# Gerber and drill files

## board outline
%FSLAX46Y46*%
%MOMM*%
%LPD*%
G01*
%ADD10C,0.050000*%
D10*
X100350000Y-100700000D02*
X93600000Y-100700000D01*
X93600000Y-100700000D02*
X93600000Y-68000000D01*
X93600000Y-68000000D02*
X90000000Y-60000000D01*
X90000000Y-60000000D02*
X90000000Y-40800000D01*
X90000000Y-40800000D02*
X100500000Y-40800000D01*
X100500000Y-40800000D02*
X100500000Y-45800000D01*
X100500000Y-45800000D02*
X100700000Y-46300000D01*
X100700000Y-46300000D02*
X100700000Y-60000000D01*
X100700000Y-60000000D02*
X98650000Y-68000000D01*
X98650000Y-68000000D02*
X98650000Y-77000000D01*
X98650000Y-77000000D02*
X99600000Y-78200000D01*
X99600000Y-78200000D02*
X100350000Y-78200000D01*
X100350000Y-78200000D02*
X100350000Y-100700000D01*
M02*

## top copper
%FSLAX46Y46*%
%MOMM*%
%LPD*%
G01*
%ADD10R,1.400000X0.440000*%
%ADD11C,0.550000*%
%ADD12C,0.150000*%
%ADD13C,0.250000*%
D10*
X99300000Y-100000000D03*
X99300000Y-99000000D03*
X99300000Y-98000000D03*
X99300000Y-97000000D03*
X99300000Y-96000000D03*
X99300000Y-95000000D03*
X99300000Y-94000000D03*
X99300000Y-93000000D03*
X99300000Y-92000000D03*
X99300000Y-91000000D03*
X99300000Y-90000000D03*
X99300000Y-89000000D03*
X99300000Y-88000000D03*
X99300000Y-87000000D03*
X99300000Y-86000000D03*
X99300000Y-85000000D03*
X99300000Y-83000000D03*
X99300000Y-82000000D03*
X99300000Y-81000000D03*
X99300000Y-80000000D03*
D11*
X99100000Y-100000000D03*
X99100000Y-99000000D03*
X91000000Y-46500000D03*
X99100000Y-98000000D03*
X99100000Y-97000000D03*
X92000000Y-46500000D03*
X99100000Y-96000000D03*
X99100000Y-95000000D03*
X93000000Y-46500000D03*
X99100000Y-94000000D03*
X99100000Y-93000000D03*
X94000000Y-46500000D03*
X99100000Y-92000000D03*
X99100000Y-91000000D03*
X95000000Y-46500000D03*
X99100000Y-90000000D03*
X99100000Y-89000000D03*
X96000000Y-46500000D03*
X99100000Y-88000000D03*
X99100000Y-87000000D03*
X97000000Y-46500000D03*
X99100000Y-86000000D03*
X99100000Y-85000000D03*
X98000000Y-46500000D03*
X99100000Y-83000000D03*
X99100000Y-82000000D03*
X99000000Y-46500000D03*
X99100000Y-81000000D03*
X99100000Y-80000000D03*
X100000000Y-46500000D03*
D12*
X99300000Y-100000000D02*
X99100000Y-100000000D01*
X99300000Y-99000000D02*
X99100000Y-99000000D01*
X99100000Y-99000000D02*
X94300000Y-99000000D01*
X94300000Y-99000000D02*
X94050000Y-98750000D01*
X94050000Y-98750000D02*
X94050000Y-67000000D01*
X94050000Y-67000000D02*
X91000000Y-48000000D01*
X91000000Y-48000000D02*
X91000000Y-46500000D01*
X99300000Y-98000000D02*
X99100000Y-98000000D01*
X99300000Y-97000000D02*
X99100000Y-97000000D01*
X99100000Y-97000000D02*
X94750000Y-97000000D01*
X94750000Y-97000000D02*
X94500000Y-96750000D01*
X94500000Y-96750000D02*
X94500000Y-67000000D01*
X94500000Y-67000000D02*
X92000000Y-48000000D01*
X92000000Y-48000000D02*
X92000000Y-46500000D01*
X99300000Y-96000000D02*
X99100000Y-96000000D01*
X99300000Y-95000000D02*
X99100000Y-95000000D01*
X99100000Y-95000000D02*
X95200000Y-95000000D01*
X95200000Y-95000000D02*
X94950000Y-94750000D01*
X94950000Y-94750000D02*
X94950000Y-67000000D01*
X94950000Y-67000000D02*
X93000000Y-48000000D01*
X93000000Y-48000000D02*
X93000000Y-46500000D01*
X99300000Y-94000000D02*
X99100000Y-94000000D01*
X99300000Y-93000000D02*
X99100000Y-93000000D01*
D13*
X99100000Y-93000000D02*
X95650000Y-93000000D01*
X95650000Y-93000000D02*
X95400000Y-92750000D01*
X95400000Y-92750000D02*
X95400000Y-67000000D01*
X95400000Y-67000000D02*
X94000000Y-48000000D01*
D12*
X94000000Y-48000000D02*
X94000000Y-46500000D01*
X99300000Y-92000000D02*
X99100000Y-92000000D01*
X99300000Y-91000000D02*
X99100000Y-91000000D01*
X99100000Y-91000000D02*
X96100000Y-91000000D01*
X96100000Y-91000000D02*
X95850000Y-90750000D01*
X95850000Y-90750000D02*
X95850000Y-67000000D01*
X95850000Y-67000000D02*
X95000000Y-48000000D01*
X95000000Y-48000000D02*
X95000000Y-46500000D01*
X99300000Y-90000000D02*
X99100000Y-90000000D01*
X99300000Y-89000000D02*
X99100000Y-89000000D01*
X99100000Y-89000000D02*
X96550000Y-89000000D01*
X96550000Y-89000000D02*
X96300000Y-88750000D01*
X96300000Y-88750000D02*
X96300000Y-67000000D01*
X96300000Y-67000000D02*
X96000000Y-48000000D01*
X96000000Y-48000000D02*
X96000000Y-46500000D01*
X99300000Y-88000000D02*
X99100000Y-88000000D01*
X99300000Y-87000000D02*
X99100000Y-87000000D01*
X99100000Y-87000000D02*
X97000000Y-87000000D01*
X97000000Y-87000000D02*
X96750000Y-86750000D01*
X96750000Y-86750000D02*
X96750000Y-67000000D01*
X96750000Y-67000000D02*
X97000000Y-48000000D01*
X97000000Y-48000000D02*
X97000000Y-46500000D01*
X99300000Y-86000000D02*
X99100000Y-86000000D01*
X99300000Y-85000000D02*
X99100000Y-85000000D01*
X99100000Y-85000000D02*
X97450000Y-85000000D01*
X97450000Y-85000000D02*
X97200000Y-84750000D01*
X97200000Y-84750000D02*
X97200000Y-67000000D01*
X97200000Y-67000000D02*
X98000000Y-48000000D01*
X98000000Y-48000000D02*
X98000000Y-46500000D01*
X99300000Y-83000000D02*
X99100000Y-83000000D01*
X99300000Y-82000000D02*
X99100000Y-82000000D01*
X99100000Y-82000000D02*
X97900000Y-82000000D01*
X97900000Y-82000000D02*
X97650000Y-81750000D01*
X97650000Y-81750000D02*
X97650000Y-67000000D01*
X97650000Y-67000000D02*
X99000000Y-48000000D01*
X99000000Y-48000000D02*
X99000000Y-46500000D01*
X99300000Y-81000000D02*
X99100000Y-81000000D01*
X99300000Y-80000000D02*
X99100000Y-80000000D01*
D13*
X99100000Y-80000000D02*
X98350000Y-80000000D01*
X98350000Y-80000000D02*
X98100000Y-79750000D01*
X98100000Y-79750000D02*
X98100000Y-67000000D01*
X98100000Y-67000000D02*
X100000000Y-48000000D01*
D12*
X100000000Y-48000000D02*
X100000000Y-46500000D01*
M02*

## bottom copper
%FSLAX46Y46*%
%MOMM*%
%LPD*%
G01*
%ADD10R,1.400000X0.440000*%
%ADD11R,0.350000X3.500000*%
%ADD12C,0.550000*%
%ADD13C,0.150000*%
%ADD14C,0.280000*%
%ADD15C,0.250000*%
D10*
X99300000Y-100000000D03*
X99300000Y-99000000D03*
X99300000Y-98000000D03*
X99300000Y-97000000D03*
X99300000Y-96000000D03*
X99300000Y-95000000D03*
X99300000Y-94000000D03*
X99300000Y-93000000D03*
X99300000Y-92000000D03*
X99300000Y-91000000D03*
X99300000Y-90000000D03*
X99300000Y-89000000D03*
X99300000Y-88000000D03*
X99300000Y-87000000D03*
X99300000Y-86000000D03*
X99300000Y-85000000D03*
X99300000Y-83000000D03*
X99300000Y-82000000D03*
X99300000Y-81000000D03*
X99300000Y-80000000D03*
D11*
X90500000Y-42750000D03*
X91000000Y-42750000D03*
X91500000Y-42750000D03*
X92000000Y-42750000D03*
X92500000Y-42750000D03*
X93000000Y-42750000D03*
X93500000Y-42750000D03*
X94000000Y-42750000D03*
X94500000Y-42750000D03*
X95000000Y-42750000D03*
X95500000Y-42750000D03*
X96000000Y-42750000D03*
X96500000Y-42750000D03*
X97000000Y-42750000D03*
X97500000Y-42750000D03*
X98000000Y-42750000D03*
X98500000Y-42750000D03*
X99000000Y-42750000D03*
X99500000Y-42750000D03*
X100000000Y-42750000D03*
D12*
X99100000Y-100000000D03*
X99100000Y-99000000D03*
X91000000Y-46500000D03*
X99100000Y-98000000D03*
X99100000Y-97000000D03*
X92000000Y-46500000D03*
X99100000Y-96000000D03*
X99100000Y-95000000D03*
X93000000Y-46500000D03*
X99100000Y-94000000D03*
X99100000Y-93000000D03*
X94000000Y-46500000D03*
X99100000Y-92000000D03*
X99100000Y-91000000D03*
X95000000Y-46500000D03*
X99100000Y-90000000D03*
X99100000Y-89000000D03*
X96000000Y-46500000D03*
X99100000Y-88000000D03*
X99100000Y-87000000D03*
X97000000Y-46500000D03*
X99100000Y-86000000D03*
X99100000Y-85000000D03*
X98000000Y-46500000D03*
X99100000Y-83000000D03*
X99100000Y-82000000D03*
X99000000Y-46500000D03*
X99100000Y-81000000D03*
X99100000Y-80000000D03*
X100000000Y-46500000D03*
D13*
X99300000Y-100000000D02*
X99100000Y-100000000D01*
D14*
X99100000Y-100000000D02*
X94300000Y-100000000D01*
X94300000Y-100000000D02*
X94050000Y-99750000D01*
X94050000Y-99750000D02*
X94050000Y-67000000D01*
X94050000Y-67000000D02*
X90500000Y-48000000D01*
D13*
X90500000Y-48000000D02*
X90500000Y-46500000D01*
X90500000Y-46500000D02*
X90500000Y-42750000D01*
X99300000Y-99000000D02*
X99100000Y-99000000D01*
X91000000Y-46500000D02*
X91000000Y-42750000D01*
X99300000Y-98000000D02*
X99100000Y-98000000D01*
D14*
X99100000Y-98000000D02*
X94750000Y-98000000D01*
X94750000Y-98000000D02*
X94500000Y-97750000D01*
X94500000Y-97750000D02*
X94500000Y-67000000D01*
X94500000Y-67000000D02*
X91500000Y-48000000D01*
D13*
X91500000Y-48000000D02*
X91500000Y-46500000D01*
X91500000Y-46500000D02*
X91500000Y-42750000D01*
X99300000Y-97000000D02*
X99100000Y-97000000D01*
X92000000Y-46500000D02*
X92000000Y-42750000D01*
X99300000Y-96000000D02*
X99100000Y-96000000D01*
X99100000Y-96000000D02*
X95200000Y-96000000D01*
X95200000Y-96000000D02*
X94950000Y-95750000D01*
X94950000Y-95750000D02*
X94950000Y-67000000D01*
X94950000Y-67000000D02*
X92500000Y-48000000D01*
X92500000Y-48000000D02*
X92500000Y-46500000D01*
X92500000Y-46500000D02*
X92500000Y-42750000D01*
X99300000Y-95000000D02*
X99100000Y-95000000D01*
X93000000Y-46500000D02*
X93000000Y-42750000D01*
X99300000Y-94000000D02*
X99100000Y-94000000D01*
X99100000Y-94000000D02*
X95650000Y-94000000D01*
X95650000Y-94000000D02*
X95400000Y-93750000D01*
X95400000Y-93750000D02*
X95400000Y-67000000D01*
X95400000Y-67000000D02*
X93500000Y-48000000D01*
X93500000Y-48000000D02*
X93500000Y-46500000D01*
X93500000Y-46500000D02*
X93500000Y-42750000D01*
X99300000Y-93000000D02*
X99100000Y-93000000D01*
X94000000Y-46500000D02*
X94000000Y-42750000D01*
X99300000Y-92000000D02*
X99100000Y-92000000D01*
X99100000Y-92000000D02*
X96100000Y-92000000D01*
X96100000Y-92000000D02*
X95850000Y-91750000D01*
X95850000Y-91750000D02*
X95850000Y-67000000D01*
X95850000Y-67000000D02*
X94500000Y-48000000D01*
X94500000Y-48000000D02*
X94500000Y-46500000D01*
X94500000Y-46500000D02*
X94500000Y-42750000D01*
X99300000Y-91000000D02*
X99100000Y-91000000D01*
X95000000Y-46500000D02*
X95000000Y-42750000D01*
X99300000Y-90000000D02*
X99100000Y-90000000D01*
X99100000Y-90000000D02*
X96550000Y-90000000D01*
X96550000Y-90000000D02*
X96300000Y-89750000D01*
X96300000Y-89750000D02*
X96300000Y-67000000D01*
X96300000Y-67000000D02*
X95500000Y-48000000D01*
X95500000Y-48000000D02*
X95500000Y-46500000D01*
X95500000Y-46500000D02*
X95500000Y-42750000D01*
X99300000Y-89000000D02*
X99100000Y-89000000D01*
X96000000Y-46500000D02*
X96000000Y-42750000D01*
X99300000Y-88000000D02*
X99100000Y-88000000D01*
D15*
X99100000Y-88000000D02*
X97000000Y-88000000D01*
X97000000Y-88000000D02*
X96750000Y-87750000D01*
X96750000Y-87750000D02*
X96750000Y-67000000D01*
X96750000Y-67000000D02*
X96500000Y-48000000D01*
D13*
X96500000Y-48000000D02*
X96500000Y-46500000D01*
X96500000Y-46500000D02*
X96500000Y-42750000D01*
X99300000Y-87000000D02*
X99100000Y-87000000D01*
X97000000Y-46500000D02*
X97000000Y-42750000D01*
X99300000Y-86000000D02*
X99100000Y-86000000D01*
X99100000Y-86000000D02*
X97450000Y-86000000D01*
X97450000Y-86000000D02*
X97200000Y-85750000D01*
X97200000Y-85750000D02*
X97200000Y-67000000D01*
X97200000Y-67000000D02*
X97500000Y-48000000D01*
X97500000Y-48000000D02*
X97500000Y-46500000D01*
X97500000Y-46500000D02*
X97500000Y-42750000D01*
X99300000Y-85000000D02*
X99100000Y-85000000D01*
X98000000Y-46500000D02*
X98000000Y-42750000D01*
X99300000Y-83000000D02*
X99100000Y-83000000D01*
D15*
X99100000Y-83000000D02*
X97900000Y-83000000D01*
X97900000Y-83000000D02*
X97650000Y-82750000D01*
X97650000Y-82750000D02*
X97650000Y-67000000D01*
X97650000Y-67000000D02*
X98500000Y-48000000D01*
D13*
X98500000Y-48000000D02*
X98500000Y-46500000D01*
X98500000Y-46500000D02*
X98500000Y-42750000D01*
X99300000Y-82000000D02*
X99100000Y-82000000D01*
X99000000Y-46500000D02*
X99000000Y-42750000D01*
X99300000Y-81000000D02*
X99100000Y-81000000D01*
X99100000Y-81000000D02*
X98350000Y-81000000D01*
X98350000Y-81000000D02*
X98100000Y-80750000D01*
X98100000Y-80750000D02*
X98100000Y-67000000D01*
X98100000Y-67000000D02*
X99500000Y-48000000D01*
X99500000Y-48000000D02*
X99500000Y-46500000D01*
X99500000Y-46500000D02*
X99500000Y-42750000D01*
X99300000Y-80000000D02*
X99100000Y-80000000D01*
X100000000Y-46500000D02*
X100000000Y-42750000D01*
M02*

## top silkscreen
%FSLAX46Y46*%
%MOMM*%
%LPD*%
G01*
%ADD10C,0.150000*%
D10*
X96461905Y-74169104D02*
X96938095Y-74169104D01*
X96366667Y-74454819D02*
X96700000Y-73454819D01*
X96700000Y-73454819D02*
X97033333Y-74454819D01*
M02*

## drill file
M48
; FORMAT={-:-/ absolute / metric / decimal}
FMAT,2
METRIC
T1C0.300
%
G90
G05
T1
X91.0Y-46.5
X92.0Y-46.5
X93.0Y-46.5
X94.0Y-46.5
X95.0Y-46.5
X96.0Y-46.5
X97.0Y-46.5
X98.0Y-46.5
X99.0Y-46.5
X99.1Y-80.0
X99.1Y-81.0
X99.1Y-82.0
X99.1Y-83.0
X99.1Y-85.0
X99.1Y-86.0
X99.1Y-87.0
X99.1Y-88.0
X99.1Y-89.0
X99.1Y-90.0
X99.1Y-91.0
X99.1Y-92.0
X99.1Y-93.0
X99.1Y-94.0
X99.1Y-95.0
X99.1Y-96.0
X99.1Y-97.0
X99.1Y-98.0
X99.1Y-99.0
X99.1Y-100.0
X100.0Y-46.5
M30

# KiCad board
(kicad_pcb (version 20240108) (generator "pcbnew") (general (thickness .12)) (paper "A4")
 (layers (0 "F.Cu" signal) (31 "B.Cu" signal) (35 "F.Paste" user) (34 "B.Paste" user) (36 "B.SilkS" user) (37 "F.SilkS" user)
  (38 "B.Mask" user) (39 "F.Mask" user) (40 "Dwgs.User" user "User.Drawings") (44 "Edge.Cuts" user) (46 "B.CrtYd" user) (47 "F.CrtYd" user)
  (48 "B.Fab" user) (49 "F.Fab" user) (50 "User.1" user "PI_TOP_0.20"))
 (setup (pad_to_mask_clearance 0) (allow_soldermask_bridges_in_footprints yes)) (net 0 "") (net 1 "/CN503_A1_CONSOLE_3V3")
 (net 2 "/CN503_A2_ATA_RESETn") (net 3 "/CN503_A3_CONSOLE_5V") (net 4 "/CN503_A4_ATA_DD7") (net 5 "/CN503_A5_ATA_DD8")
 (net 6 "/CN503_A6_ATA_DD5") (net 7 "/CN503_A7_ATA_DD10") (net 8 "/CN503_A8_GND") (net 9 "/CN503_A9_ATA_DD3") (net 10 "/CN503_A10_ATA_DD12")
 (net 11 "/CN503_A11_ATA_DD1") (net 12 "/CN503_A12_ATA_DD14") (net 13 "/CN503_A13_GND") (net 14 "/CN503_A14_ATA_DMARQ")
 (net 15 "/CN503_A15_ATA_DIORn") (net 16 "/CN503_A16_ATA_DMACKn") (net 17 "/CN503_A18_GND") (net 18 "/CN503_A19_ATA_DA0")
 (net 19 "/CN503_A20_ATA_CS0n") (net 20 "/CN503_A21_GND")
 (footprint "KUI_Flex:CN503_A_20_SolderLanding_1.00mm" (layer "F.Cu") (at 100.0 100.0)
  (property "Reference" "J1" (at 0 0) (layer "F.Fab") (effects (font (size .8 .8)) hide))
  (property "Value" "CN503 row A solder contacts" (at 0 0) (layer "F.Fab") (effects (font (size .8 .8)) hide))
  (pad "1" smd rect (at -0.7 0) (size 1.4 .44) (layers "F.Cu" "F.Mask") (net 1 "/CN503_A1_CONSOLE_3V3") (solder_mask_margin .29))
  (pad "1" smd rect (at -0.7 0) (size 1.4 .44) (layers "B.Cu" "B.Mask") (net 1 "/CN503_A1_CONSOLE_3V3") (solder_mask_margin .29))
  (pad "2" smd rect (at -0.7 -1) (size 1.4 .44) (layers "F.Cu" "F.Mask") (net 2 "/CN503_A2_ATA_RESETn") (solder_mask_margin .29))
  (pad "2" smd rect (at -0.7 -1) (size 1.4 .44) (layers "B.Cu" "B.Mask") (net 2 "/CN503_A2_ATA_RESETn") (solder_mask_margin .29))
  (pad "3" smd rect (at -0.7 -2) (size 1.4 .44) (layers "F.Cu" "F.Mask") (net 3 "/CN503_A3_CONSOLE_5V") (solder_mask_margin .29))
  (pad "3" smd rect (at -0.7 -2) (size 1.4 .44) (layers "B.Cu" "B.Mask") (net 3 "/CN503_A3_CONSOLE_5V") (solder_mask_margin .29))
  (pad "4" smd rect (at -0.7 -3) (size 1.4 .44) (layers "F.Cu" "F.Mask") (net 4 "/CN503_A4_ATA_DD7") (solder_mask_margin .29))
  (pad "4" smd rect (at -0.7 -3) (size 1.4 .44) (layers "B.Cu" "B.Mask") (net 4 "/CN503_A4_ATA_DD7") (solder_mask_margin .29))
  (pad "5" smd rect (at -0.7 -4) (size 1.4 .44) (layers "F.Cu" "F.Mask") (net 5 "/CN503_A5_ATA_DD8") (solder_mask_margin .29))
  (pad "5" smd rect (at -0.7 -4) (size 1.4 .44) (layers "B.Cu" "B.Mask") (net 5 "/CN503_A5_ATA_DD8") (solder_mask_margin .29))
  (pad "6" smd rect (at -0.7 -5) (size 1.4 .44) (layers "F.Cu" "F.Mask") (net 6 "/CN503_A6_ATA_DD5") (solder_mask_margin .29))
  (pad "6" smd rect (at -0.7 -5) (size 1.4 .44) (layers "B.Cu" "B.Mask") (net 6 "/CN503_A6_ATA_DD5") (solder_mask_margin .29))
  (pad "7" smd rect (at -0.7 -6) (size 1.4 .44) (layers "F.Cu" "F.Mask") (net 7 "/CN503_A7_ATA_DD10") (solder_mask_margin .29))
  (pad "7" smd rect (at -0.7 -6) (size 1.4 .44) (layers "B.Cu" "B.Mask") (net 7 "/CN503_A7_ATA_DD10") (solder_mask_margin .29))
  (pad "8" smd rect (at -0.7 -7) (size 1.4 .44) (layers "F.Cu" "F.Mask") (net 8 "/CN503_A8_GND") (solder_mask_margin .29))
  (pad "8" smd rect (at -0.7 -7) (size 1.4 .44) (layers "B.Cu" "B.Mask") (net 8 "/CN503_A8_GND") (solder_mask_margin .29))
  (pad "9" smd rect (at -0.7 -8) (size 1.4 .44) (layers "F.Cu" "F.Mask") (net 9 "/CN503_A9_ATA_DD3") (solder_mask_margin .29))
  (pad "9" smd rect (at -0.7 -8) (size 1.4 .44) (layers "B.Cu" "B.Mask") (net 9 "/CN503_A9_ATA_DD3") (solder_mask_margin .29))
  (pad "10" smd rect (at -0.7 -9) (size 1.4 .44) (layers "F.Cu" "F.Mask") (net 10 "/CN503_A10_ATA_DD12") (solder_mask_margin .29))
  (pad "10" smd rect (at -0.7 -9) (size 1.4 .44) (layers "B.Cu" "B.Mask") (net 10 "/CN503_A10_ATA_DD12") (solder_mask_margin .29))
  (pad "11" smd rect (at -0.7 -10) (size 1.4 .44) (layers "F.Cu" "F.Mask") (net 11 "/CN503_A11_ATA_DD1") (solder_mask_margin .29))
  (pad "11" smd rect (at -0.7 -10) (size 1.4 .44) (layers "B.Cu" "B.Mask") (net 11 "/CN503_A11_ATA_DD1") (solder_mask_margin .29))
  (pad "12" smd rect (at -0.7 -11) (size 1.4 .44) (layers "F.Cu" "F.Mask") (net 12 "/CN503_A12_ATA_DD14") (solder_mask_margin .29))
  (pad "12" smd rect (at -0.7 -11) (size 1.4 .44) (layers "B.Cu" "B.Mask") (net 12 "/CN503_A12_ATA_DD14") (solder_mask_margin .29))
  (pad "13" smd rect (at -0.7 -12) (size 1.4 .44) (layers "F.Cu" "F.Mask") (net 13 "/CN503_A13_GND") (solder_mask_margin .29))
  (pad "13" smd rect (at -0.7 -12) (size 1.4 .44) (layers "B.Cu" "B.Mask") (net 13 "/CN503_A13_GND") (solder_mask_margin .29))
  (pad "14" smd rect (at -0.7 -13) (size 1.4 .44) (layers "F.Cu" "F.Mask") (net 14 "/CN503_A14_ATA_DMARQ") (solder_mask_margin .29))
  (pad "14" smd rect (at -0.7 -13) (size 1.4 .44) (layers "B.Cu" "B.Mask") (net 14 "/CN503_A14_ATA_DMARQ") (solder_mask_margin .29))
  (pad "15" smd rect (at -0.7 -14) (size 1.4 .44) (layers "F.Cu" "F.Mask") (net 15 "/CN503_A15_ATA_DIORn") (solder_mask_margin .29))
  (pad "15" smd rect (at -0.7 -14) (size 1.4 .44) (layers "B.Cu" "B.Mask") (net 15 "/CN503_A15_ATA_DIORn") (solder_mask_margin .29))
  (pad "16" smd rect (at -0.7 -15) (size 1.4 .44) (layers "F.Cu" "F.Mask") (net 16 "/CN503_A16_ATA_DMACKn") (solder_mask_margin .29))
  (pad "16" smd rect (at -0.7 -15) (size 1.4 .44) (layers "B.Cu" "B.Mask") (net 16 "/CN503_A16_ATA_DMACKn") (solder_mask_margin .29))
  (pad "18" smd rect (at -0.7 -17) (size 1.4 .44) (layers "F.Cu" "F.Mask") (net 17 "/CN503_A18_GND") (solder_mask_margin .29))
  (pad "18" smd rect (at -0.7 -17) (size 1.4 .44) (layers "B.Cu" "B.Mask") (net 17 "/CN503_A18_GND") (solder_mask_margin .29))
  (pad "19" smd rect (at -0.7 -18) (size 1.4 .44) (layers "F.Cu" "F.Mask") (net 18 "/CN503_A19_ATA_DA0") (solder_mask_margin .29))
  (pad "19" smd rect (at -0.7 -18) (size 1.4 .44) (layers "B.Cu" "B.Mask") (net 18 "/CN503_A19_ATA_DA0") (solder_mask_margin .29))
  (pad "20" smd rect (at -0.7 -19) (size 1.4 .44) (layers "F.Cu" "F.Mask") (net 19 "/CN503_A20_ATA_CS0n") (solder_mask_margin .29))
  (pad "20" smd rect (at -0.7 -19) (size 1.4 .44) (layers "B.Cu" "B.Mask") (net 19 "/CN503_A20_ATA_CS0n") (solder_mask_margin .29))
  (pad "21" smd rect (at -0.7 -20) (size 1.4 .44) (layers "F.Cu" "F.Mask") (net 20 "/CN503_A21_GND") (solder_mask_margin .29))
  (pad "21" smd rect (at -0.7 -20) (size 1.4 .44) (layers "B.Cu" "B.Mask") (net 20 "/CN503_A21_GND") (solder_mask_margin .29)))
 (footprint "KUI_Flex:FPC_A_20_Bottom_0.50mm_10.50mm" (layer "F.Cu") (at 100.0 100.0)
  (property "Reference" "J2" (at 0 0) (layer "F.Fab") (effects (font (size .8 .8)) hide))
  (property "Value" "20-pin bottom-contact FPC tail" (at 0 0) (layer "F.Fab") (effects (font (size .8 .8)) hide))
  (pad "1" smd rect (at -9.5 -57.25) (size .35 3.5) (layers "B.Cu" "B.Mask") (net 1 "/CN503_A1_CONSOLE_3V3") (solder_mask_margin .10))
  (pad "2" smd rect (at -9 -57.25) (size .35 3.5) (layers "B.Cu" "B.Mask") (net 2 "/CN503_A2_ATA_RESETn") (solder_mask_margin .10))
  (pad "3" smd rect (at -8.5 -57.25) (size .35 3.5) (layers "B.Cu" "B.Mask") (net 3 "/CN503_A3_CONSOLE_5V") (solder_mask_margin .10))
  (pad "4" smd rect (at -8 -57.25) (size .35 3.5) (layers "B.Cu" "B.Mask") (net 4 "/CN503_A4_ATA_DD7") (solder_mask_margin .10))
  (pad "5" smd rect (at -7.5 -57.25) (size .35 3.5) (layers "B.Cu" "B.Mask") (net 5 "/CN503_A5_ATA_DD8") (solder_mask_margin .10))
  (pad "6" smd rect (at -7 -57.25) (size .35 3.5) (layers "B.Cu" "B.Mask") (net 6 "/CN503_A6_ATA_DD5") (solder_mask_margin .10))
  (pad "7" smd rect (at -6.5 -57.25) (size .35 3.5) (layers "B.Cu" "B.Mask") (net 7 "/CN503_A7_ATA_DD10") (solder_mask_margin .10))
  (pad "8" smd rect (at -6 -57.25) (size .35 3.5) (layers "B.Cu" "B.Mask") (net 8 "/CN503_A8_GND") (solder_mask_margin .10))
  (pad "9" smd rect (at -5.5 -57.25) (size .35 3.5) (layers "B.Cu" "B.Mask") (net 9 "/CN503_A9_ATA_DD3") (solder_mask_margin .10))
  (pad "10" smd rect (at -5 -57.25) (size .35 3.5) (layers "B.Cu" "B.Mask") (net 10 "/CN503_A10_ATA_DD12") (solder_mask_margin .10))
  (pad "11" smd rect (at -4.5 -57.25) (size .35 3.5) (layers "B.Cu" "B.Mask") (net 11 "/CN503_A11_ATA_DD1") (solder_mask_margin .10))
  (pad "12" smd rect (at -4 -57.25) (size .35 3.5) (layers "B.Cu" "B.Mask") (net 12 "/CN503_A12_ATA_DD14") (solder_mask_margin .10))
  (pad "13" smd rect (at -3.5 -57.25) (size .35 3.5) (layers "B.Cu" "B.Mask") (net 13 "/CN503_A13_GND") (solder_mask_margin .10))
  (pad "14" smd rect (at -3 -57.25) (size .35 3.5) (layers "B.Cu" "B.Mask") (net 14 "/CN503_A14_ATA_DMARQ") (solder_mask_margin .10))
  (pad "15" smd rect (at -2.5 -57.25) (size .35 3.5) (layers "B.Cu" "B.Mask") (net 15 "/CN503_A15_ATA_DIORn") (solder_mask_margin .10))
  (pad "16" smd rect (at -2 -57.25) (size .35 3.5) (layers "B.Cu" "B.Mask") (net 16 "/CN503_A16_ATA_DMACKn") (solder_mask_margin .10))
  (pad "17" smd rect (at -1.5 -57.25) (size .35 3.5) (layers "B.Cu" "B.Mask") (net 17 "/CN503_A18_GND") (solder_mask_margin .10))
  (pad "18" smd rect (at -1 -57.25) (size .35 3.5) (layers "B.Cu" "B.Mask") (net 18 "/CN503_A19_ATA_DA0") (solder_mask_margin .10))
  (pad "19" smd rect (at -0.5 -57.25) (size .35 3.5) (layers "B.Cu" "B.Mask") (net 19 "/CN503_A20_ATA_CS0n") (solder_mask_margin .10))
  (pad "20" smd rect (at -0 -57.25) (size .35 3.5) (layers "B.Cu" "B.Mask") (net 20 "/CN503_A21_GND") (solder_mask_margin .10)))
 (segment (start 99.3 100) (end 99.1 100) (width 0.15) (layer "F.Cu") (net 1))
 (segment (start 99.3 100) (end 99.1 100) (width 0.15) (layer "B.Cu") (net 1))
 (segment (start 99.1 100) (end 94.3 100) (width 0.28) (layer "B.Cu") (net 1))
 (segment (start 94.3 100) (end 94.05 99.75) (width 0.28) (layer "B.Cu") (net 1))
 (segment (start 94.05 99.75) (end 94.05 67) (width 0.28) (layer "B.Cu") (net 1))
 (segment (start 94.05 67) (end 90.5 48) (width 0.28) (layer "B.Cu") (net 1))
 (segment (start 90.5 48) (end 90.5 46.5) (width 0.15) (layer "B.Cu") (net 1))
 (segment (start 90.5 46.5) (end 90.5 42.75) (width 0.15) (layer "B.Cu") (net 1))
 (segment (start 99.3 99) (end 99.1 99) (width 0.15) (layer "F.Cu") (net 2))
 (segment (start 99.3 99) (end 99.1 99) (width 0.15) (layer "B.Cu") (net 2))
 (segment (start 99.1 99) (end 94.3 99) (width 0.15) (layer "F.Cu") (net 2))
 (segment (start 94.3 99) (end 94.05 98.75) (width 0.15) (layer "F.Cu") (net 2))
 (segment (start 94.05 98.75) (end 94.05 67) (width 0.15) (layer "F.Cu") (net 2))
 (segment (start 94.05 67) (end 91 48) (width 0.15) (layer "F.Cu") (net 2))
 (segment (start 91 48) (end 91 46.5) (width 0.15) (layer "F.Cu") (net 2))
 (segment (start 91 46.5) (end 91 42.75) (width 0.15) (layer "B.Cu") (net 2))
 (segment (start 99.3 98) (end 99.1 98) (width 0.15) (layer "F.Cu") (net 3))
 (segment (start 99.3 98) (end 99.1 98) (width 0.15) (layer "B.Cu") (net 3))
 (segment (start 99.1 98) (end 94.75 98) (width 0.28) (layer "B.Cu") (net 3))
 (segment (start 94.75 98) (end 94.5 97.75) (width 0.28) (layer "B.Cu") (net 3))
 (segment (start 94.5 97.75) (end 94.5 67) (width 0.28) (layer "B.Cu") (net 3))
 (segment (start 94.5 67) (end 91.5 48) (width 0.28) (layer "B.Cu") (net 3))
 (segment (start 91.5 48) (end 91.5 46.5) (width 0.15) (layer "B.Cu") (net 3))
 (segment (start 91.5 46.5) (end 91.5 42.75) (width 0.15) (layer "B.Cu") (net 3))
 (segment (start 99.3 97) (end 99.1 97) (width 0.15) (layer "F.Cu") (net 4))
 (segment (start 99.3 97) (end 99.1 97) (width 0.15) (layer "B.Cu") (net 4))
 (segment (start 99.1 97) (end 94.75 97) (width 0.15) (layer "F.Cu") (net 4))
 (segment (start 94.75 97) (end 94.5 96.75) (width 0.15) (layer "F.Cu") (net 4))
 (segment (start 94.5 96.75) (end 94.5 67) (width 0.15) (layer "F.Cu") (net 4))
 (segment (start 94.5 67) (end 92 48) (width 0.15) (layer "F.Cu") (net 4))
 (segment (start 92 48) (end 92 46.5) (width 0.15) (layer "F.Cu") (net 4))
 (segment (start 92 46.5) (end 92 42.75) (width 0.15) (layer "B.Cu") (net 4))
 (segment (start 99.3 96) (end 99.1 96) (width 0.15) (layer "F.Cu") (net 5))
 (segment (start 99.3 96) (end 99.1 96) (width 0.15) (layer "B.Cu") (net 5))
 (segment (start 99.1 96) (end 95.2 96) (width 0.15) (layer "B.Cu") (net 5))
 (segment (start 95.2 96) (end 94.95 95.75) (width 0.15) (layer "B.Cu") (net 5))
 (segment (start 94.95 95.75) (end 94.95 67) (width 0.15) (layer "B.Cu") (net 5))
 (segment (start 94.95 67) (end 92.5 48) (width 0.15) (layer "B.Cu") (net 5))
 (segment (start 92.5 48) (end 92.5 46.5) (width 0.15) (layer "B.Cu") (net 5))
 (segment (start 92.5 46.5) (end 92.5 42.75) (width 0.15) (layer "B.Cu") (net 5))
 (segment (start 99.3 95) (end 99.1 95) (width 0.15) (layer "F.Cu") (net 6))
 (segment (start 99.3 95) (end 99.1 95) (width 0.15) (layer "B.Cu") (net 6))
 (segment (start 99.1 95) (end 95.2 95) (width 0.15) (layer "F.Cu") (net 6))
 (segment (start 95.2 95) (end 94.95 94.75) (width 0.15) (layer "F.Cu") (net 6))
 (segment (start 94.95 94.75) (end 94.95 67) (width 0.15) (layer "F.Cu") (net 6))
 (segment (start 94.95 67) (end 93 48) (width 0.15) (layer "F.Cu") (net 6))
 (segment (start 93 48) (end 93 46.5) (width 0.15) (layer "F.Cu") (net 6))
 (segment (start 93 46.5) (end 93 42.75) (width 0.15) (layer "B.Cu") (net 6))
 (segment (start 99.3 94) (end 99.1 94) (width 0.15) (layer "F.Cu") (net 7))
 (segment (start 99.3 94) (end 99.1 94) (width 0.15) (layer "B.Cu") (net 7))
 (segment (start 99.1 94) (end 95.65 94) (width 0.15) (layer "B.Cu") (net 7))
 (segment (start 95.65 94) (end 95.4 93.75) (width 0.15) (layer "B.Cu") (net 7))
 (segment (start 95.4 93.75) (end 95.4 67) (width 0.15) (layer "B.Cu") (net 7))
 (segment (start 95.4 67) (end 93.5 48) (width 0.15) (layer "B.Cu") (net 7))
 (segment (start 93.5 48) (end 93.5 46.5) (width 0.15) (layer "B.Cu") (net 7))
 (segment (start 93.5 46.5) (end 93.5 42.75) (width 0.15) (layer "B.Cu") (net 7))
 (segment (start 99.3 93) (end 99.1 93) (width 0.15) (layer "F.Cu") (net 8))
 (segment (start 99.3 93) (end 99.1 93) (width 0.15) (layer "B.Cu") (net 8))
 (segment (start 99.1 93) (end 95.65 93) (width 0.25) (layer "F.Cu") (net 8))
 (segment (start 95.65 93) (end 95.4 92.75) (width 0.25) (layer "F.Cu") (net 8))
 (segment (start 95.4 92.75) (end 95.4 67) (width 0.25) (layer "F.Cu") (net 8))
 (segment (start 95.4 67) (end 94 48) (width 0.25) (layer "F.Cu") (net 8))
 (segment (start 94 48) (end 94 46.5) (width 0.15) (layer "F.Cu") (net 8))
 (segment (start 94 46.5) (end 94 42.75) (width 0.15) (layer "B.Cu") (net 8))
 (segment (start 99.3 92) (end 99.1 92) (width 0.15) (layer "F.Cu") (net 9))
 (segment (start 99.3 92) (end 99.1 92) (width 0.15) (layer "B.Cu") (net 9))
 (segment (start 99.1 92) (end 96.1 92) (width 0.15) (layer "B.Cu") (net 9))
 (segment (start 96.1 92) (end 95.85 91.75) (width 0.15) (layer "B.Cu") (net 9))
 (segment (start 95.85 91.75) (end 95.85 67) (width 0.15) (layer "B.Cu") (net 9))
 (segment (start 95.85 67) (end 94.5 48) (width 0.15) (layer "B.Cu") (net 9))
 (segment (start 94.5 48) (end 94.5 46.5) (width 0.15) (layer "B.Cu") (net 9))
 (segment (start 94.5 46.5) (end 94.5 42.75) (width 0.15) (layer "B.Cu") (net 9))
 (segment (start 99.3 91) (end 99.1 91) (width 0.15) (layer "F.Cu") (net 10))
 (segment (start 99.3 91) (end 99.1 91) (width 0.15) (layer "B.Cu") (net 10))
 (segment (start 99.1 91) (end 96.1 91) (width 0.15) (layer "F.Cu") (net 10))
 (segment (start 96.1 91) (end 95.85 90.75) (width 0.15) (layer "F.Cu") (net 10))
 (segment (start 95.85 90.75) (end 95.85 67) (width 0.15) (layer "F.Cu") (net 10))
 (segment (start 95.85 67) (end 95 48) (width 0.15) (layer "F.Cu") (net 10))
 (segment (start 95 48) (end 95 46.5) (width 0.15) (layer "F.Cu") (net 10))
 (segment (start 95 46.5) (end 95 42.75) (width 0.15) (layer "B.Cu") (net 10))
 (segment (start 99.3 90) (end 99.1 90) (width 0.15) (layer "F.Cu") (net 11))
 (segment (start 99.3 90) (end 99.1 90) (width 0.15) (layer "B.Cu") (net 11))
 (segment (start 99.1 90) (end 96.55 90) (width 0.15) (layer "B.Cu") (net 11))
 (segment (start 96.55 90) (end 96.3 89.75) (width 0.15) (layer "B.Cu") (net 11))
 (segment (start 96.3 89.75) (end 96.3 67) (width 0.15) (layer "B.Cu") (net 11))
 (segment (start 96.3 67) (end 95.5 48) (width 0.15) (layer "B.Cu") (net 11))
 (segment (start 95.5 48) (end 95.5 46.5) (width 0.15) (layer "B.Cu") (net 11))
 (segment (start 95.5 46.5) (end 95.5 42.75) (width 0.15) (layer "B.Cu") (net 11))
 (segment (start 99.3 89) (end 99.1 89) (width 0.15) (layer "F.Cu") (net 12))
 (segment (start 99.3 89) (end 99.1 89) (width 0.15) (layer "B.Cu") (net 12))
 (segment (start 99.1 89) (end 96.55 89) (width 0.15) (layer "F.Cu") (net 12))
 (segment (start 96.55 89) (end 96.3 88.75) (width 0.15) (layer "F.Cu") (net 12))
 (segment (start 96.3 88.75) (end 96.3 67) (width 0.15) (layer "F.Cu") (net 12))
 (segment (start 96.3 67) (end 96 48) (width 0.15) (layer "F.Cu") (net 12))
 (segment (start 96 48) (end 96 46.5) (width 0.15) (layer "F.Cu") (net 12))
 (segment (start 96 46.5) (end 96 42.75) (width 0.15) (layer "B.Cu") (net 12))
 (segment (start 99.3 88) (end 99.1 88) (width 0.15) (layer "F.Cu") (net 13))
 (segment (start 99.3 88) (end 99.1 88) (width 0.15) (layer "B.Cu") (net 13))
 (segment (start 99.1 88) (end 97 88) (width 0.25) (layer "B.Cu") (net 13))
 (segment (start 97 88) (end 96.75 87.75) (width 0.25) (layer "B.Cu") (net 13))
 (segment (start 96.75 87.75) (end 96.75 67) (width 0.25) (layer "B.Cu") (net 13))
 (segment (start 96.75 67) (end 96.5 48) (width 0.25) (layer "B.Cu") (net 13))
 (segment (start 96.5 48) (end 96.5 46.5) (width 0.15) (layer "B.Cu") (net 13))
 (segment (start 96.5 46.5) (end 96.5 42.75) (width 0.15) (layer "B.Cu") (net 13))
 (segment (start 99.3 87) (end 99.1 87) (width 0.15) (layer "F.Cu") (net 14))
 (segment (start 99.3 87) (end 99.1 87) (width 0.15) (layer "B.Cu") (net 14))
 (segment (start 99.1 87) (end 97 87) (width 0.15) (layer "F.Cu") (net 14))
 (segment (start 97 87) (end 96.75 86.75) (width 0.15) (layer "F.Cu") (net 14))
 (segment (start 96.75 86.75) (end 96.75 67) (width 0.15) (layer "F.Cu") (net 14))
 (segment (start 96.75 67) (end 97 48) (width 0.15) (layer "F.Cu") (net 14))
 (segment (start 97 48) (end 97 46.5) (width 0.15) (layer "F.Cu") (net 14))
 (segment (start 97 46.5) (end 97 42.75) (width 0.15) (layer "B.Cu") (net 14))
 (segment (start 99.3 86) (end 99.1 86) (width 0.15) (layer "F.Cu") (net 15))
 (segment (start 99.3 86) (end 99.1 86) (width 0.15) (layer "B.Cu") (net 15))
 (segment (start 99.1 86) (end 97.45 86) (width 0.15) (layer "B.Cu") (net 15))
 (segment (start 97.45 86) (end 97.2 85.75) (width 0.15) (layer "B.Cu") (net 15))
 (segment (start 97.2 85.75) (end 97.2 67) (width 0.15) (layer "B.Cu") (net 15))
 (segment (start 97.2 67) (end 97.5 48) (width 0.15) (layer "B.Cu") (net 15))
 (segment (start 97.5 48) (end 97.5 46.5) (width 0.15) (layer "B.Cu") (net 15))
 (segment (start 97.5 46.5) (end 97.5 42.75) (width 0.15) (layer "B.Cu") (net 15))
 (segment (start 99.3 85) (end 99.1 85) (width 0.15) (layer "F.Cu") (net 16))
 (segment (start 99.3 85) (end 99.1 85) (width 0.15) (layer "B.Cu") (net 16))
 (segment (start 99.1 85) (end 97.45 85) (width 0.15) (layer "F.Cu") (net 16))
 (segment (start 97.45 85) (end 97.2 84.75) (width 0.15) (layer "F.Cu") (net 16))
 (segment (start 97.2 84.75) (end 97.2 67) (width 0.15) (layer "F.Cu") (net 16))
 (segment (start 97.2 67) (end 98 48) (width 0.15) (layer "F.Cu") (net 16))
 (segment (start 98 48) (end 98 46.5) (width 0.15) (layer "F.Cu") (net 16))
 (segment (start 98 46.5) (end 98 42.75) (width 0.15) (layer "B.Cu") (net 16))
 (segment (start 99.3 83) (end 99.1 83) (width 0.15) (layer "F.Cu") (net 17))
 (segment (start 99.3 83) (end 99.1 83) (width 0.15) (layer "B.Cu") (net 17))
 (segment (start 99.1 83) (end 97.9 83) (width 0.25) (layer "B.Cu") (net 17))
 (segment (start 97.9 83) (end 97.65 82.75) (width 0.25) (layer "B.Cu") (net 17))
 (segment (start 97.65 82.75) (end 97.65 67) (width 0.25) (layer "B.Cu") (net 17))
 (segment (start 97.65 67) (end 98.5 48) (width 0.25) (layer "B.Cu") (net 17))
 (segment (start 98.5 48) (end 98.5 46.5) (width 0.15) (layer "B.Cu") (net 17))
 (segment (start 98.5 46.5) (end 98.5 42.75) (width 0.15) (layer "B.Cu") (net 17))
 (segment (start 99.3 82) (end 99.1 82) (width 0.15) (layer "F.Cu") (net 18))
 (segment (start 99.3 82) (end 99.1 82) (width 0.15) (layer "B.Cu") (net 18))
 (segment (start 99.1 82) (end 97.9 82) (width 0.15) (layer "F.Cu") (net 18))
 (segment (start 97.9 82) (end 97.65 81.75) (width 0.15) (layer "F.Cu") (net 18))
 (segment (start 97.65 81.75) (end 97.65 67) (width 0.15) (layer "F.Cu") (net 18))
 (segment (start 97.65 67) (end 99 48) (width 0.15) (layer "F.Cu") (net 18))
 (segment (start 99 48) (end 99 46.5) (width 0.15) (layer "F.Cu") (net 18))
 (segment (start 99 46.5) (end 99 42.75) (width 0.15) (layer "B.Cu") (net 18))
 (segment (start 99.3 81) (end 99.1 81) (width 0.15) (layer "F.Cu") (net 19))
 (segment (start 99.3 81) (end 99.1 81) (width 0.15) (layer "B.Cu") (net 19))
 (segment (start 99.1 81) (end 98.35 81) (width 0.15) (layer "B.Cu") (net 19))
 (segment (start 98.35 81) (end 98.1 80.75) (width 0.15) (layer "B.Cu") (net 19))
 (segment (start 98.1 80.75) (end 98.1 67) (width 0.15) (layer "B.Cu") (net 19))
 (segment (start 98.1 67) (end 99.5 48) (width 0.15) (layer "B.Cu") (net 19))
 (segment (start 99.5 48) (end 99.5 46.5) (width 0.15) (layer "B.Cu") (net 19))
 (segment (start 99.5 46.5) (end 99.5 42.75) (width 0.15) (layer "B.Cu") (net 19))
 (segment (start 99.3 80) (end 99.1 80) (width 0.15) (layer "F.Cu") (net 20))
 (segment (start 99.3 80) (end 99.1 80) (width 0.15) (layer "B.Cu") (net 20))
 (segment (start 99.1 80) (end 98.35 80) (width 0.25) (layer "F.Cu") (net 20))
 (segment (start 98.35 80) (end 98.1 79.75) (width 0.25) (layer "F.Cu") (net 20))
 (segment (start 98.1 79.75) (end 98.1 67) (width 0.25) (layer "F.Cu") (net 20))
 (segment (start 98.1 67) (end 100 48) (width 0.25) (layer "F.Cu") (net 20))
 (segment (start 100 48) (end 100 46.5) (width 0.15) (layer "F.Cu") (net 20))
 (segment (start 100 46.5) (end 100 42.75) (width 0.15) (layer "B.Cu") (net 20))
 (via (at 99.1 100) (size .55) (drill .3) (layers "F.Cu" "B.Cu") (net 1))
 (via (at 99.1 99) (size .55) (drill .3) (layers "F.Cu" "B.Cu") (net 2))
 (via (at 91 46.5) (size .55) (drill .3) (layers "F.Cu" "B.Cu") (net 2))
 (via (at 99.1 98) (size .55) (drill .3) (layers "F.Cu" "B.Cu") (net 3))
 (via (at 99.1 97) (size .55) (drill .3) (layers "F.Cu" "B.Cu") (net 4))
 (via (at 92 46.5) (size .55) (drill .3) (layers "F.Cu" "B.Cu") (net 4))
 (via (at 99.1 96) (size .55) (drill .3) (layers "F.Cu" "B.Cu") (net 5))
 (via (at 99.1 95) (size .55) (drill .3) (layers "F.Cu" "B.Cu") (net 6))
 (via (at 93 46.5) (size .55) (drill .3) (layers "F.Cu" "B.Cu") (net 6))
 (via (at 99.1 94) (size .55) (drill .3) (layers "F.Cu" "B.Cu") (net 7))
 (via (at 99.1 93) (size .55) (drill .3) (layers "F.Cu" "B.Cu") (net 8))
 (via (at 94 46.5) (size .55) (drill .3) (layers "F.Cu" "B.Cu") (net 8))
 (via (at 99.1 92) (size .55) (drill .3) (layers "F.Cu" "B.Cu") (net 9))
 (via (at 99.1 91) (size .55) (drill .3) (layers "F.Cu" "B.Cu") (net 10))
 (via (at 95 46.5) (size .55) (drill .3) (layers "F.Cu" "B.Cu") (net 10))
 (via (at 99.1 90) (size .55) (drill .3) (layers "F.Cu" "B.Cu") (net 11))
 (via (at 99.1 89) (size .55) (drill .3) (layers "F.Cu" "B.Cu") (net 12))
 (via (at 96 46.5) (size .55) (drill .3) (layers "F.Cu" "B.Cu") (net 12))
 (via (at 99.1 88) (size .55) (drill .3) (layers "F.Cu" "B.Cu") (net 13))
 (via (at 99.1 87) (size .55) (drill .3) (layers "F.Cu" "B.Cu") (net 14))
 (via (at 97 46.5) (size .55) (drill .3) (layers "F.Cu" "B.Cu") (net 14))
 (via (at 99.1 86) (size .55) (drill .3) (layers "F.Cu" "B.Cu") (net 15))
 (via (at 99.1 85) (size .55) (drill .3) (layers "F.Cu" "B.Cu") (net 16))
 (via (at 98 46.5) (size .55) (drill .3) (layers "F.Cu" "B.Cu") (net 16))
 (via (at 99.1 83) (size .55) (drill .3) (layers "F.Cu" "B.Cu") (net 17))
 (via (at 99.1 82) (size .55) (drill .3) (layers "F.Cu" "B.Cu") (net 18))
 (via (at 99 46.5) (size .55) (drill .3) (layers "F.Cu" "B.Cu") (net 18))
 (via (at 99.1 81) (size .55) (drill .3) (layers "F.Cu" "B.Cu") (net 19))
 (via (at 99.1 80) (size .55) (drill .3) (layers "F.Cu" "B.Cu") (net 20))
 (via (at 100 46.5) (size .55) (drill .3) (layers "F.Cu" "B.Cu") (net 20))
 (gr_line (start 100.35 100.7) (end 93.6 100.7) (stroke (width .05) (type default)) (layer "Edge.Cuts"))
 (gr_line (start 93.6 100.7) (end 93.6 68) (stroke (width .05) (type default)) (layer "Edge.Cuts"))
 (gr_line (start 93.6 68) (end 90 60) (stroke (width .05) (type default)) (layer "Edge.Cuts"))
 (gr_line (start 90 60) (end 90 40.8) (stroke (width .05) (type default)) (layer "Edge.Cuts"))
 (gr_line (start 90 40.8) (end 100.5 40.8) (stroke (width .05) (type default)) (layer "Edge.Cuts"))
 (gr_line (start 100.5 40.8) (end 100.5 45.8) (stroke (width .05) (type default)) (layer "Edge.Cuts"))
 (gr_line (start 100.5 45.8) (end 100.7 46.3) (stroke (width .05) (type default)) (layer "Edge.Cuts"))
 (gr_line (start 100.7 46.3) (end 100.7 60) (stroke (width .05) (type default)) (layer "Edge.Cuts"))
 (gr_line (start 100.7 60) (end 98.65 68) (stroke (width .05) (type default)) (layer "Edge.Cuts"))
 (gr_line (start 98.65 68) (end 98.65 77) (stroke (width .05) (type default)) (layer "Edge.Cuts"))
 (gr_line (start 98.65 77) (end 99.6 78.2) (stroke (width .05) (type default)) (layer "Edge.Cuts"))
 (gr_line (start 99.6 78.2) (end 100.35 78.2) (stroke (width .05) (type default)) (layer "Edge.Cuts"))
 (gr_line (start 100.35 78.2) (end 100.35 100.7) (stroke (width .05) (type default)) (layer "Edge.Cuts"))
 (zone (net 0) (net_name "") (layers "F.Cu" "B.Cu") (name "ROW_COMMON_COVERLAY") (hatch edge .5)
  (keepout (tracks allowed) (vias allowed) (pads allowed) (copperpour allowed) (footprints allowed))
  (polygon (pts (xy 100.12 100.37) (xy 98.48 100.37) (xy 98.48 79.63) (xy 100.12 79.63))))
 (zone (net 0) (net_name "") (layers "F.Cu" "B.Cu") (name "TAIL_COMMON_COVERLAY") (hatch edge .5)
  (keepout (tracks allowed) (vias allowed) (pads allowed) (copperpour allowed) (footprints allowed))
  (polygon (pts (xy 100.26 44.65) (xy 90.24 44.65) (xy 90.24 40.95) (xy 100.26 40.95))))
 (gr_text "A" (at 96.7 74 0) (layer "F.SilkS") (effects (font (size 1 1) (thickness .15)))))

